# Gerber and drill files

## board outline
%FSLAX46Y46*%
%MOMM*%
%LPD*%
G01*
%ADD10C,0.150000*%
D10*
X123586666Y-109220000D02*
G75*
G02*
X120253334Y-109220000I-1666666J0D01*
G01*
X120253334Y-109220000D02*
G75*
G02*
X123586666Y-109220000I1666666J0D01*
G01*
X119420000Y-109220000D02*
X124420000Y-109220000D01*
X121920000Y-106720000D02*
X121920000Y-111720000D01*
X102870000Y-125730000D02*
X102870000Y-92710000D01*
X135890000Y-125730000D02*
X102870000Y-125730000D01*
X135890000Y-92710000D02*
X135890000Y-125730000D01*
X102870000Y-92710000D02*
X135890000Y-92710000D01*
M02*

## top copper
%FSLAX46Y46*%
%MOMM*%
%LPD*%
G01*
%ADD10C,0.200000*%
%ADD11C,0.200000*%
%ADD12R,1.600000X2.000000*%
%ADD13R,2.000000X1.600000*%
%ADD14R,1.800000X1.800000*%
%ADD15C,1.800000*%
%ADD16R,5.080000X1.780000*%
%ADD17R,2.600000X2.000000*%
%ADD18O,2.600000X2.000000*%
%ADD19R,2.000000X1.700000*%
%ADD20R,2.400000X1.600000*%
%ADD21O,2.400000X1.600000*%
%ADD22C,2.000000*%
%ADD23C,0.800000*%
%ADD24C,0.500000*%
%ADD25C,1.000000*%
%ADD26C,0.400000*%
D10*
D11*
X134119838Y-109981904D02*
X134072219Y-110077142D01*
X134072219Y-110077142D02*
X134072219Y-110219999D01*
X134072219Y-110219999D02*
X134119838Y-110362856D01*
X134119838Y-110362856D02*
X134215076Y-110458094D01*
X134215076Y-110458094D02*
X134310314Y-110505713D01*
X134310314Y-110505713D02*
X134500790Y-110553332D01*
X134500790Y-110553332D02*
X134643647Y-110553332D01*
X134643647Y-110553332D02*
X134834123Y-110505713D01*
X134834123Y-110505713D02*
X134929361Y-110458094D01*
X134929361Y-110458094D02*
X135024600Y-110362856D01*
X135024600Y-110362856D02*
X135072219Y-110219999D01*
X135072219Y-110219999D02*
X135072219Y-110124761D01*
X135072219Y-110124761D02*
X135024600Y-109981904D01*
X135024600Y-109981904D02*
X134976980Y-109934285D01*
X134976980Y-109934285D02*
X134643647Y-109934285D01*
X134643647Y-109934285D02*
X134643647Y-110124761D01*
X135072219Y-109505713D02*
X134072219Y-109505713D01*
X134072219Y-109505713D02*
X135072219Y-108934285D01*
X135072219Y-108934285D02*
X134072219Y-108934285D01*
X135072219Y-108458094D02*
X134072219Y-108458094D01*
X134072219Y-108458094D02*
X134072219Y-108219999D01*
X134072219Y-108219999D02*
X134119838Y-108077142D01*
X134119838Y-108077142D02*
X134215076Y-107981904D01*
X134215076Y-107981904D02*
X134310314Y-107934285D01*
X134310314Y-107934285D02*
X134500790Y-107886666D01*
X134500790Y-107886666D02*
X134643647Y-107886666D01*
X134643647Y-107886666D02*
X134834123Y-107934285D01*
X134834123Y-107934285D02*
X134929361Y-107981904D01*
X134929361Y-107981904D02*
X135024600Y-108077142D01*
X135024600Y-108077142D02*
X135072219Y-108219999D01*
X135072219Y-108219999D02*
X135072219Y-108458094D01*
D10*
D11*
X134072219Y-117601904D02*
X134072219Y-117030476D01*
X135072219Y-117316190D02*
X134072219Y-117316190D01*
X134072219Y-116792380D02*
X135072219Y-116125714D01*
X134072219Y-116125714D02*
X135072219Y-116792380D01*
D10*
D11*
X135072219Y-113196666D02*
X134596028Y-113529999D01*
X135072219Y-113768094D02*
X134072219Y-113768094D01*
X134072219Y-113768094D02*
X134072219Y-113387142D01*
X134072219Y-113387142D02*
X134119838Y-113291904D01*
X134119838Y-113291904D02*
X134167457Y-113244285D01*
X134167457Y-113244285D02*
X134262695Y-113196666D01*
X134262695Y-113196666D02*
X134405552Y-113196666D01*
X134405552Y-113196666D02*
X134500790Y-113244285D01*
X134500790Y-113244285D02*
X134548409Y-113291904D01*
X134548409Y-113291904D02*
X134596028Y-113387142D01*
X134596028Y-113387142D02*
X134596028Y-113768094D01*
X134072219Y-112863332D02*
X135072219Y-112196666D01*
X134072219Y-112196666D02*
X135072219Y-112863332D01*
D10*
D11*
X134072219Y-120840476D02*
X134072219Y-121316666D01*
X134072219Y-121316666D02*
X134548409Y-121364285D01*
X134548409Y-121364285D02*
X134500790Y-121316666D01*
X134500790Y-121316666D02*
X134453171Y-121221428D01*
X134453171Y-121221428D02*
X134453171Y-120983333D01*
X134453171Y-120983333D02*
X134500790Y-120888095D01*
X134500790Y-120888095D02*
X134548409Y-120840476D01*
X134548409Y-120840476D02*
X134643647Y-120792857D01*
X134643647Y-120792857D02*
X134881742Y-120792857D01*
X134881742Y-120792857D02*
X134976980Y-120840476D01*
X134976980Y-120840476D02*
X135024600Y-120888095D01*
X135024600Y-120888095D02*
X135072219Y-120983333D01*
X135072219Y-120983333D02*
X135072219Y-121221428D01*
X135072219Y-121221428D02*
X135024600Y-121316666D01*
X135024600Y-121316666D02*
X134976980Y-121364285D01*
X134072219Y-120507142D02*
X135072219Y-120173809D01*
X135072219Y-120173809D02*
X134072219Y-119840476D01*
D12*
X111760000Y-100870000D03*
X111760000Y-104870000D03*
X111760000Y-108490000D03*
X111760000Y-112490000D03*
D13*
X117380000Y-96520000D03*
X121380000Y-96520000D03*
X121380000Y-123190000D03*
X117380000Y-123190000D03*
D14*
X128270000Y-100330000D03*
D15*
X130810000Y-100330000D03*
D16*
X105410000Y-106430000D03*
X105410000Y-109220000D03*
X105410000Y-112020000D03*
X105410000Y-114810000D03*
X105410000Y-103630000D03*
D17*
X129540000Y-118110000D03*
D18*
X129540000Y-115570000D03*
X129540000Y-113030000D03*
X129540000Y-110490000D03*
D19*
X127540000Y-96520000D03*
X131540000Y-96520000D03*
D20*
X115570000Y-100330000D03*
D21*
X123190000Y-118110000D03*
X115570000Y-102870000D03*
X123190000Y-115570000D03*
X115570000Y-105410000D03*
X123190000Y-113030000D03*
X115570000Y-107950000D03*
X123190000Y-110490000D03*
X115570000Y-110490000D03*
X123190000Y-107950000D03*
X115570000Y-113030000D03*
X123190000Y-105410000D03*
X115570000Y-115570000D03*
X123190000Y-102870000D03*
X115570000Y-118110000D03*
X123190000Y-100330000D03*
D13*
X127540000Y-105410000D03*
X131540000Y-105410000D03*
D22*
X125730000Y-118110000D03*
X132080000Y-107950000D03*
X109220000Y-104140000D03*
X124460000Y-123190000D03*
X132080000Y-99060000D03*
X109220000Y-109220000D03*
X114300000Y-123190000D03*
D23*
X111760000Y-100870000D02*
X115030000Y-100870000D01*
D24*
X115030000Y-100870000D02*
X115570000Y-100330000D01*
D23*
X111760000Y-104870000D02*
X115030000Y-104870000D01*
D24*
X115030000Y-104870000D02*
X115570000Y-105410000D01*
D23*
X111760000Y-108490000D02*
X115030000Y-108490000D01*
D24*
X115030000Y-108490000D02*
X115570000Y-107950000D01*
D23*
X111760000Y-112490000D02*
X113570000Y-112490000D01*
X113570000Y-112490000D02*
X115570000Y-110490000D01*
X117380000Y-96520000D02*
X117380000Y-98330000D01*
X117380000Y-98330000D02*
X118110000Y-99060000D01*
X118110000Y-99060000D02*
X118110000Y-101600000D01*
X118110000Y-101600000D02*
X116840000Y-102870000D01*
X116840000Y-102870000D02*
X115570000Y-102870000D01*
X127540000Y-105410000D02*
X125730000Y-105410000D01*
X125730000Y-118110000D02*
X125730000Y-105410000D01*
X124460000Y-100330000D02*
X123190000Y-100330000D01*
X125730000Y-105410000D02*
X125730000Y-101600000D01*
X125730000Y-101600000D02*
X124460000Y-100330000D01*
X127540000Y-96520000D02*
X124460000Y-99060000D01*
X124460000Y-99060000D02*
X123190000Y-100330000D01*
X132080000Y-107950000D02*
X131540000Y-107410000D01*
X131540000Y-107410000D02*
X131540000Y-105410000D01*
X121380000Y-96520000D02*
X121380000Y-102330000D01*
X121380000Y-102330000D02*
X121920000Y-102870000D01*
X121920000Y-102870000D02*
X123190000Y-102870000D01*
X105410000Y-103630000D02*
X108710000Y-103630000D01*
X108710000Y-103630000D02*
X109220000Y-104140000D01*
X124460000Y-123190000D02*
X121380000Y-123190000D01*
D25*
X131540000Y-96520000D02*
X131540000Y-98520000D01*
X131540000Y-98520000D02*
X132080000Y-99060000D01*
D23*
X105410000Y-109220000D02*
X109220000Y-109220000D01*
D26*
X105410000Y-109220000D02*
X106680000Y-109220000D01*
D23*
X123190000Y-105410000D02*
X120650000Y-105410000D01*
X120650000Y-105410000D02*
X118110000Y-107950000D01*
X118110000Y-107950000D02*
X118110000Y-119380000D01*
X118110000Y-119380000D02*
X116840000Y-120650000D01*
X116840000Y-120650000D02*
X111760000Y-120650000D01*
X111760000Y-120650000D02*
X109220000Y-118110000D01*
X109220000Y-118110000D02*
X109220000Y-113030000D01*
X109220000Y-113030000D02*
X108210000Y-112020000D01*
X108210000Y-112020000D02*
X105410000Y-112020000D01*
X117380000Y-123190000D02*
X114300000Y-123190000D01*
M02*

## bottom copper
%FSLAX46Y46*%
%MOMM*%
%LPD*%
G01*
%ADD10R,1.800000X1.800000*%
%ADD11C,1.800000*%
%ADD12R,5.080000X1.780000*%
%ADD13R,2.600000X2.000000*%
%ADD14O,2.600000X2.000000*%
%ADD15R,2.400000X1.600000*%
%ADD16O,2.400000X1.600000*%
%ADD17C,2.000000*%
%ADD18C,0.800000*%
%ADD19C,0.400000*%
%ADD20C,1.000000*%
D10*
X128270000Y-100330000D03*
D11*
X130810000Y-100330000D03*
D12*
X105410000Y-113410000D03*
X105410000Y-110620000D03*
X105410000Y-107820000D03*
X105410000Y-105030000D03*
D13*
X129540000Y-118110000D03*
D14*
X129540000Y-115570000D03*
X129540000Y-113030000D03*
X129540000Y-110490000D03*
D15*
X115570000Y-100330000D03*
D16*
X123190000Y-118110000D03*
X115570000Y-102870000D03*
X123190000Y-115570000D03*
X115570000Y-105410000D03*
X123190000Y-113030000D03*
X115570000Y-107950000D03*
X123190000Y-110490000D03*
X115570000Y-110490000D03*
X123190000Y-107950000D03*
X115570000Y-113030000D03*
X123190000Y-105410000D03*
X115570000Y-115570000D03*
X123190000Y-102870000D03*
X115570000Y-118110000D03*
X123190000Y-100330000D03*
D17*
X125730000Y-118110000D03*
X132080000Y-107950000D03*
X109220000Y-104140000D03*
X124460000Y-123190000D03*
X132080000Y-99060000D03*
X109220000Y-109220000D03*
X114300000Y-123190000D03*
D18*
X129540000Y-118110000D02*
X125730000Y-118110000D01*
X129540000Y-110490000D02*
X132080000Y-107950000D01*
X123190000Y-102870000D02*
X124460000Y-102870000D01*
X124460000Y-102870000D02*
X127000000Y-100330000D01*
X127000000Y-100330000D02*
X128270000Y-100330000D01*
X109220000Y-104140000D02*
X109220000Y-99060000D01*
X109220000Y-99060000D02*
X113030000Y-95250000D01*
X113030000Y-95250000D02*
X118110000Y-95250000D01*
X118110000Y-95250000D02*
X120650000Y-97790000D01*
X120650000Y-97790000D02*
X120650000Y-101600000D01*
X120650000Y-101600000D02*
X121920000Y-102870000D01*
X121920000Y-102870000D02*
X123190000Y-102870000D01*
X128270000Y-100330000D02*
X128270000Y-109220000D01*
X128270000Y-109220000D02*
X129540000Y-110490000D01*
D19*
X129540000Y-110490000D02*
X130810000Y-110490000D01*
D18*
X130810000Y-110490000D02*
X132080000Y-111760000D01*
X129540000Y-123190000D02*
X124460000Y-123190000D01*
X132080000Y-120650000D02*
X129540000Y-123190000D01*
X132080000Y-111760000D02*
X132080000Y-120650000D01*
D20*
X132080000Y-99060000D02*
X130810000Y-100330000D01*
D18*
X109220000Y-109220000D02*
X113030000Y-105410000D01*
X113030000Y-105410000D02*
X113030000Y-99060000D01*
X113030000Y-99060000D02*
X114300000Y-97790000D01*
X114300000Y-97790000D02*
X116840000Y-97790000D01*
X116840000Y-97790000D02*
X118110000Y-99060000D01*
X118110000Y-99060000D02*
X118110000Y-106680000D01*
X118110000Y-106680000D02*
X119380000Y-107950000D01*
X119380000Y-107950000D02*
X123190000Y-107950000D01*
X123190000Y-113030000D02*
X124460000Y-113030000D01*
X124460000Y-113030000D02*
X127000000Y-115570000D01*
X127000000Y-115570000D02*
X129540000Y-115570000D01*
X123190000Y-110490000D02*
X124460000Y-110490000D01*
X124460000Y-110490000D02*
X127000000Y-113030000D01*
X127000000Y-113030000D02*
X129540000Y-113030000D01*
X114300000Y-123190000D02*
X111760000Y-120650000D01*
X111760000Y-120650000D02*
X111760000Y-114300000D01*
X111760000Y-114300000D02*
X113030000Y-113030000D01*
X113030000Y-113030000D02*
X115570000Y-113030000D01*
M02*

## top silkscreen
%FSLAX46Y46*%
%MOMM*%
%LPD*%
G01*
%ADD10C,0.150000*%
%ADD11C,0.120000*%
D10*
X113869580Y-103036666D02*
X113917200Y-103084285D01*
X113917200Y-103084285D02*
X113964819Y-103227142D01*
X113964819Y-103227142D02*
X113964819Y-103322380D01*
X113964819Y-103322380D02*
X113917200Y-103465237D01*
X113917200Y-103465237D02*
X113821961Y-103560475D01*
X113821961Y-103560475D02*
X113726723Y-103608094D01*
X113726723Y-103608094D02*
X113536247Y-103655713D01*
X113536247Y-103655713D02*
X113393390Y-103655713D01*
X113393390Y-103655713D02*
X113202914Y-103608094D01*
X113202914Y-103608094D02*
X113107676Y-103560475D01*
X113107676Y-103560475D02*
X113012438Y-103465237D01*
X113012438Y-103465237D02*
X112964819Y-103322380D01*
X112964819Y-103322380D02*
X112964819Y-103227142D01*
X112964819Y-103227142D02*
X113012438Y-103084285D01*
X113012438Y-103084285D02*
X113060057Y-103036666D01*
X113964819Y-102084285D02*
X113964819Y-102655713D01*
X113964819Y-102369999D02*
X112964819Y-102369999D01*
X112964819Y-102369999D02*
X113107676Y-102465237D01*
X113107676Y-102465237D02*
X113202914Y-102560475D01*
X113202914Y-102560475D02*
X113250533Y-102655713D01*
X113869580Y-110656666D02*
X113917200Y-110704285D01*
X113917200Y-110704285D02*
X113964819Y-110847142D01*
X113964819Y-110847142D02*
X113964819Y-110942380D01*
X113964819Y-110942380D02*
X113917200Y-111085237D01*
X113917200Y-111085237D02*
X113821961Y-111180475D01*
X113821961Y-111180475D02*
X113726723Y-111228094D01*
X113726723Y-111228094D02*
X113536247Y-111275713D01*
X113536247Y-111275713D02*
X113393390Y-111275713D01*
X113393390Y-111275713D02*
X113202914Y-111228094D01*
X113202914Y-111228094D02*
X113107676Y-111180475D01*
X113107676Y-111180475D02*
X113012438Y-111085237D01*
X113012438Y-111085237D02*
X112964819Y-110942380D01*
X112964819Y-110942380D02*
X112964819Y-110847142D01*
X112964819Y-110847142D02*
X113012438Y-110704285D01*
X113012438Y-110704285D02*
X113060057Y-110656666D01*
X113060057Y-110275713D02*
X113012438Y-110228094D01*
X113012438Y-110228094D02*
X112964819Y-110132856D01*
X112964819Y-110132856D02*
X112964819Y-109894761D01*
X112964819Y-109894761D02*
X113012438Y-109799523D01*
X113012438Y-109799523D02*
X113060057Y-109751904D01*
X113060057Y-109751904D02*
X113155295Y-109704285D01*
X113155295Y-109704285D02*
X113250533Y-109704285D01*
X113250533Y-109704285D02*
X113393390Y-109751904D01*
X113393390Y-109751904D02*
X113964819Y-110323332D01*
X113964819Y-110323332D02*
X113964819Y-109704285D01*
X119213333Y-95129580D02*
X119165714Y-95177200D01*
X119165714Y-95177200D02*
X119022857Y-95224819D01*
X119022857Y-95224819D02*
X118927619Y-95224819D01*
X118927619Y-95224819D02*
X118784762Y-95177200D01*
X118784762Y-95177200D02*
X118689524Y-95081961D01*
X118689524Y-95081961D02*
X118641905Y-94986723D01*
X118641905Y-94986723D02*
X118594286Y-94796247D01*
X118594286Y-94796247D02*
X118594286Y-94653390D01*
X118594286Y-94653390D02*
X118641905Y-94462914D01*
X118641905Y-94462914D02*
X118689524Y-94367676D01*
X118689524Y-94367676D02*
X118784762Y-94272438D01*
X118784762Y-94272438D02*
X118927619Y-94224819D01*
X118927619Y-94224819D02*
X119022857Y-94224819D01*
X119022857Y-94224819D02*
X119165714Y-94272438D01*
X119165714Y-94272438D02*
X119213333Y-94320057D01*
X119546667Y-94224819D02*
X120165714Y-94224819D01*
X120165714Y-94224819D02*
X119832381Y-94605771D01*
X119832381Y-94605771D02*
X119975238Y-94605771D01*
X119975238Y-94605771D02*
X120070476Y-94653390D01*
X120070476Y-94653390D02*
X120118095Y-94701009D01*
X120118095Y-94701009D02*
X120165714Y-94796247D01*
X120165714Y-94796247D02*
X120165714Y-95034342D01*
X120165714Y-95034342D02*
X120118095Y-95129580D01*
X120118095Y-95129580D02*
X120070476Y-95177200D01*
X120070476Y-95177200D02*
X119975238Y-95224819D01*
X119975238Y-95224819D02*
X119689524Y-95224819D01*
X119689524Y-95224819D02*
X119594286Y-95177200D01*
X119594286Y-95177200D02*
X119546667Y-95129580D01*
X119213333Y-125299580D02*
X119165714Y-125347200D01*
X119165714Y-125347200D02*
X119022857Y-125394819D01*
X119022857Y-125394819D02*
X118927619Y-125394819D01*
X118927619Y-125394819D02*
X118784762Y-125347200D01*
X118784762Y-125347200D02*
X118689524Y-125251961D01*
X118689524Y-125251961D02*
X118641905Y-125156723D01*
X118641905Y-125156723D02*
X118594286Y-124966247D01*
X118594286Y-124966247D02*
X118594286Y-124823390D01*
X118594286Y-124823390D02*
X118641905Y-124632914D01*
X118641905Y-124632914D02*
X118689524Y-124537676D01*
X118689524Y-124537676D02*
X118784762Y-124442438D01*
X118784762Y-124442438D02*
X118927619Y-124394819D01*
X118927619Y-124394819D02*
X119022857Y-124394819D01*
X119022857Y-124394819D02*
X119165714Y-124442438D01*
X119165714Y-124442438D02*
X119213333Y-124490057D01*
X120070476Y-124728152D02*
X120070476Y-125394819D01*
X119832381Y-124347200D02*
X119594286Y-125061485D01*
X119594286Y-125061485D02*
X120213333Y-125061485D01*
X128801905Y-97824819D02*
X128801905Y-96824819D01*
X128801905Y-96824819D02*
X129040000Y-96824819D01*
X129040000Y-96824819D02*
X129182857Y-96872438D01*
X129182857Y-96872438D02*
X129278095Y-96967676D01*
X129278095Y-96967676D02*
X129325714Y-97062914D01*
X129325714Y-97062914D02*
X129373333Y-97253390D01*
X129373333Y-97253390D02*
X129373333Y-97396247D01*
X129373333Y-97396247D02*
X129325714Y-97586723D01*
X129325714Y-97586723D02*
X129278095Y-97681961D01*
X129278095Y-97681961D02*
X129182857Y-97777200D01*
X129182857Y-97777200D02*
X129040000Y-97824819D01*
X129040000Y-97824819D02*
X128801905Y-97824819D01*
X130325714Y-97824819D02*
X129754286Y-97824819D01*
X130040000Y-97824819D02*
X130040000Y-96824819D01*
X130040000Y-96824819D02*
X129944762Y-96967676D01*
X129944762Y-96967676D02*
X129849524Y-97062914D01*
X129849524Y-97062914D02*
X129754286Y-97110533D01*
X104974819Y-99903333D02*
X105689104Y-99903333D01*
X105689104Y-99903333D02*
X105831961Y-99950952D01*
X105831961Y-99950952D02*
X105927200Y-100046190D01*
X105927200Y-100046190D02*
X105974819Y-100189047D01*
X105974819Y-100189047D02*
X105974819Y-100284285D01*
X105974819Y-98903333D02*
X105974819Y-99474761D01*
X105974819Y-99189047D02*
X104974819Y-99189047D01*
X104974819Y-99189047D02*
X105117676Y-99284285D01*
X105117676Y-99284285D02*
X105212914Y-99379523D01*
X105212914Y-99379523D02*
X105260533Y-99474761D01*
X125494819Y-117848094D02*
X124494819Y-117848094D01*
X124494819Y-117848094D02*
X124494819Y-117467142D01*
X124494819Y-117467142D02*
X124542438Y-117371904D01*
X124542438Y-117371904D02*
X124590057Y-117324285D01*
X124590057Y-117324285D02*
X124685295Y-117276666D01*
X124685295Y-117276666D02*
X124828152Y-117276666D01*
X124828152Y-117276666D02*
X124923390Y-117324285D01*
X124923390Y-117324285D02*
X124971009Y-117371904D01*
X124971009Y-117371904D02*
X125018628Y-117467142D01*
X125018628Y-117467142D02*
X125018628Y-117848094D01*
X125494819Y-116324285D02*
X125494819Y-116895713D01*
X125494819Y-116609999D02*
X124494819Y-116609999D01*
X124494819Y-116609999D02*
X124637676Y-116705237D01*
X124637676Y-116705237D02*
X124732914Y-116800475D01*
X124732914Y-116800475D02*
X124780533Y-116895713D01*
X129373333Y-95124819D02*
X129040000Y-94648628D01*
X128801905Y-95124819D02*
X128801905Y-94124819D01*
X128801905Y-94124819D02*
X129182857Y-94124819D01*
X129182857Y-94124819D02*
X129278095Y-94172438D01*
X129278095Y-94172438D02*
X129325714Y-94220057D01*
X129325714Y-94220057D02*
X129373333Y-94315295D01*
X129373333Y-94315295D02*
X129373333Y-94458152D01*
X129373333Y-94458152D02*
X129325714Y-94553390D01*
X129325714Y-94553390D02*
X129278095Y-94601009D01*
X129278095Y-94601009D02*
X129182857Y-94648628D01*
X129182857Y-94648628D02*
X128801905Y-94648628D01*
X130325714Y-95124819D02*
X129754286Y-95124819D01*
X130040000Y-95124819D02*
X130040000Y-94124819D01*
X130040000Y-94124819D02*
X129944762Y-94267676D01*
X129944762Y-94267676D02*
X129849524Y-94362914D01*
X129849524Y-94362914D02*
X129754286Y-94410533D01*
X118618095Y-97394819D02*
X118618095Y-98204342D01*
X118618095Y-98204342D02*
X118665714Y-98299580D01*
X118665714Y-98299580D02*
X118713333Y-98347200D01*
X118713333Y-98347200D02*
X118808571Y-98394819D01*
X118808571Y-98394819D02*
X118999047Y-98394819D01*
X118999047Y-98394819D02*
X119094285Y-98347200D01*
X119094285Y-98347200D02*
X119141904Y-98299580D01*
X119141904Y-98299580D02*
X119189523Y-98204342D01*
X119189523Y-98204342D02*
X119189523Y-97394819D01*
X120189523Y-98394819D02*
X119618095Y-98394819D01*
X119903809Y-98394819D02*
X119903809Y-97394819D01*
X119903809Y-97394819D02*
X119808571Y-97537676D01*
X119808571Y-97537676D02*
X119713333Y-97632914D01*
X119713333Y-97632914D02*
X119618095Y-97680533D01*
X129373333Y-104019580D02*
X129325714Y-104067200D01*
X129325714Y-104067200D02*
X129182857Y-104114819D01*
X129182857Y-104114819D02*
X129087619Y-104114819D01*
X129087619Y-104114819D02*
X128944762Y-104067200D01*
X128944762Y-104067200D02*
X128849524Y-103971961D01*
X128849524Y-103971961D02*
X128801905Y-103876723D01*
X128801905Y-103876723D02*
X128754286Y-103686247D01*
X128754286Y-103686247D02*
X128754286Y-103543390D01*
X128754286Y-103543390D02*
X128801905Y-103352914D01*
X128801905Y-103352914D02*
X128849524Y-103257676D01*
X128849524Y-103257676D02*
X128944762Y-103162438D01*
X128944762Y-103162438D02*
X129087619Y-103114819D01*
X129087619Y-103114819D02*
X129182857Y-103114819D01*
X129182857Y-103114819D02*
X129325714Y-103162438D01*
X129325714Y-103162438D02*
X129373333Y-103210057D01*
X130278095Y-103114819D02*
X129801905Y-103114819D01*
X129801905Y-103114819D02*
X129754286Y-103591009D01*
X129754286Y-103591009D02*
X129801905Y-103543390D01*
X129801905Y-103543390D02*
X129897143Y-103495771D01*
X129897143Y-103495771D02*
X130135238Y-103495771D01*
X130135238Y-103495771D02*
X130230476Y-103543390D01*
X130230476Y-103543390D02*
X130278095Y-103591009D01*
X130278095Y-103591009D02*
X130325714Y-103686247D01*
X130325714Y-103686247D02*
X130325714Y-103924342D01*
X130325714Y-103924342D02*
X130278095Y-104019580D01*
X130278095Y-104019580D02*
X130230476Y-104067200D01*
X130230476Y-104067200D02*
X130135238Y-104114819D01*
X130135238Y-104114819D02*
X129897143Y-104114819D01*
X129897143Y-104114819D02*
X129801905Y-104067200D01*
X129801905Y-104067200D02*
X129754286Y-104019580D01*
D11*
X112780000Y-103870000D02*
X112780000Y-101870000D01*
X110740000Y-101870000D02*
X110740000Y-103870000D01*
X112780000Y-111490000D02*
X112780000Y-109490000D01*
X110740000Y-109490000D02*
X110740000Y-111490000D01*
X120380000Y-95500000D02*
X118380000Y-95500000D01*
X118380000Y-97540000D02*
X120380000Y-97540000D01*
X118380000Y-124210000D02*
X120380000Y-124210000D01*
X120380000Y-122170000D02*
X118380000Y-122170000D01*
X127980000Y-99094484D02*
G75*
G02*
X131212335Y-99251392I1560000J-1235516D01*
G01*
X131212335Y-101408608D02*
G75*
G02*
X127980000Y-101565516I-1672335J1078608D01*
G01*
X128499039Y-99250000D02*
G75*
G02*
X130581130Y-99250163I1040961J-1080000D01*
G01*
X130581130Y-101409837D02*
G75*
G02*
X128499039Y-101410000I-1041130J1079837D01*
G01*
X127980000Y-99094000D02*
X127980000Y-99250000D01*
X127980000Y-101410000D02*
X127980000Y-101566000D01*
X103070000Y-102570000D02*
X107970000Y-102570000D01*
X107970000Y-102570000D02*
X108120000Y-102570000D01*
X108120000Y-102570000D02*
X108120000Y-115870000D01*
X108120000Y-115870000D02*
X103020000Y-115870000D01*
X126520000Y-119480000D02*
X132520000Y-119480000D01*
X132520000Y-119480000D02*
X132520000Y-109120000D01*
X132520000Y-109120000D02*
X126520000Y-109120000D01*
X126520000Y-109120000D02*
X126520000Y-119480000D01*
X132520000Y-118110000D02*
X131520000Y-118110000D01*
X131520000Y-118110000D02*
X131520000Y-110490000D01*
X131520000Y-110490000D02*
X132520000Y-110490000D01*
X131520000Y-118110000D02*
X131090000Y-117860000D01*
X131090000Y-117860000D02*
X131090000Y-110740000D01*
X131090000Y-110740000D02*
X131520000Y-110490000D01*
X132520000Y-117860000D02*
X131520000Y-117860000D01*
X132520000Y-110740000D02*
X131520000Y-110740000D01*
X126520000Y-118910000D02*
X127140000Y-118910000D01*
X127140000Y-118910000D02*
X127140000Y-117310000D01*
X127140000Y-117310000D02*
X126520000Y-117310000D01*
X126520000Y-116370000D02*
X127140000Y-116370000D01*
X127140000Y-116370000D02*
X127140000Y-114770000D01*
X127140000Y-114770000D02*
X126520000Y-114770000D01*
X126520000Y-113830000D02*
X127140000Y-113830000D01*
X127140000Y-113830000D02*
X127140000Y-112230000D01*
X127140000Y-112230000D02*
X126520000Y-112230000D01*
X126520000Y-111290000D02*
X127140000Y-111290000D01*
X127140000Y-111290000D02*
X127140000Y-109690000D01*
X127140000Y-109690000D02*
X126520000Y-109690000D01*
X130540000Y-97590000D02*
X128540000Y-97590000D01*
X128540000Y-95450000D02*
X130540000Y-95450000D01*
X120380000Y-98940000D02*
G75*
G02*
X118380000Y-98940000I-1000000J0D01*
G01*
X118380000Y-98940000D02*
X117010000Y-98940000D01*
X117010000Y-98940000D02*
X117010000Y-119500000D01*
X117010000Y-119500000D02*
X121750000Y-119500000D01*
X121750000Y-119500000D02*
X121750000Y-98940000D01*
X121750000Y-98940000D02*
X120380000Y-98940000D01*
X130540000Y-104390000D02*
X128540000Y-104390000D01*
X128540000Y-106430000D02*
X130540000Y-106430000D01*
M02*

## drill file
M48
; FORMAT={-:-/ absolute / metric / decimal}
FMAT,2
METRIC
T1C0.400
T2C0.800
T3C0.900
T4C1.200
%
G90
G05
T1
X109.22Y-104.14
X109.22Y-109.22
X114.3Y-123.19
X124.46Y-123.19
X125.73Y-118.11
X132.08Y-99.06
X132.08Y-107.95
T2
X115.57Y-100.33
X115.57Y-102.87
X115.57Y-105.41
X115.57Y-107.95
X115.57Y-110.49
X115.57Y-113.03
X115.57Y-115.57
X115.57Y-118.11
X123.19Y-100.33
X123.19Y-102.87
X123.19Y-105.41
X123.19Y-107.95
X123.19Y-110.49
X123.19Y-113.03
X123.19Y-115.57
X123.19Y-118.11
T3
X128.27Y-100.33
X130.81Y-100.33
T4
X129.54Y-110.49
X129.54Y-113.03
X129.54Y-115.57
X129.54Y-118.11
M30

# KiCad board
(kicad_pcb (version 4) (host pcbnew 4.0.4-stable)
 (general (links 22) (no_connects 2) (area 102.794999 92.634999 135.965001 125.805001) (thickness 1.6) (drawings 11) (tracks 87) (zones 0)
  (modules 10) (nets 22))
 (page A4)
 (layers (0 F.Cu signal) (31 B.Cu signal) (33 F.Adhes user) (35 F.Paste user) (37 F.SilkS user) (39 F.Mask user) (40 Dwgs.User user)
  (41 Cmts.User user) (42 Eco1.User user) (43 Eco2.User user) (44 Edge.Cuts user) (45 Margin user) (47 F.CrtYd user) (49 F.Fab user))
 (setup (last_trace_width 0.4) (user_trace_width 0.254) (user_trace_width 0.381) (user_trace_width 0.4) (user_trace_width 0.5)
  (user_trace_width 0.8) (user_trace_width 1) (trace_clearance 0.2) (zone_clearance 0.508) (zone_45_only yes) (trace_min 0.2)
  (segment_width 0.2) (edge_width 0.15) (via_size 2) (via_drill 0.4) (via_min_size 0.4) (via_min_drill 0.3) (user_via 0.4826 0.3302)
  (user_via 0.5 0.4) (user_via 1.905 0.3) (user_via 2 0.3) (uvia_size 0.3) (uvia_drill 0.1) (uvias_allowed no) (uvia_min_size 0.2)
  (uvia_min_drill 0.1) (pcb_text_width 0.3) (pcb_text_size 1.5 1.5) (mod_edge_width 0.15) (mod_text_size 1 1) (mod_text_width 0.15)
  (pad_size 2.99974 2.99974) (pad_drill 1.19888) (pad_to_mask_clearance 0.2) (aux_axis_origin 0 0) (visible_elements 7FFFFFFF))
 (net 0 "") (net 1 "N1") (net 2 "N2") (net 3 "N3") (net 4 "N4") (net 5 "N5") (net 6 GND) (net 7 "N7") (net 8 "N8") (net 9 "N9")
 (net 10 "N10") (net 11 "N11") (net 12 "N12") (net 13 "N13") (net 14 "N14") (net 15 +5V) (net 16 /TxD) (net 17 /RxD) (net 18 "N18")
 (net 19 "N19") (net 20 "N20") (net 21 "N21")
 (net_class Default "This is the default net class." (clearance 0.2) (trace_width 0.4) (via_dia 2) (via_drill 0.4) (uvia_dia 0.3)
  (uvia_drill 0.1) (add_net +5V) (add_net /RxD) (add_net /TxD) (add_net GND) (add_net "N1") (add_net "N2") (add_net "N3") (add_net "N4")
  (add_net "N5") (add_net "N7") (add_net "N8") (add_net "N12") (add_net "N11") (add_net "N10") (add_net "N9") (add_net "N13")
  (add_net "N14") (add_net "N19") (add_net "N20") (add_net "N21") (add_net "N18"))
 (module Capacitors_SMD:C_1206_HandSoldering (layer F.Cu) (at 111.76 102.87 270)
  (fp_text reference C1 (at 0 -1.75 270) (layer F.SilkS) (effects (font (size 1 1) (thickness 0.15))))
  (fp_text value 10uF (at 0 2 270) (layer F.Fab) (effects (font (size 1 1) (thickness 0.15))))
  (fp_line (start 1 -1.02) (end -1 -1.02) (layer F.SilkS) (width 0.12))
  (fp_line (start -1 1.02) (end 1 1.02) (layer F.SilkS) (width 0.12))
  (pad 1 smd rect (at -2 0 270) (size 2 1.6) (layers F.Cu F.Paste F.Mask) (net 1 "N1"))
  (pad 2 smd rect (at 2 0 270) (size 2 1.6) (layers F.Cu F.Paste F.Mask) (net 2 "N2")))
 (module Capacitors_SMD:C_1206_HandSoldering (layer F.Cu) (at 111.76 110.49 270)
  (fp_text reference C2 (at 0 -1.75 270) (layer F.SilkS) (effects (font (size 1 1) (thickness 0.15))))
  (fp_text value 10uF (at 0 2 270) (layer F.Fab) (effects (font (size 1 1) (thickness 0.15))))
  (fp_line (start 1 -1.02) (end -1 -1.02) (layer F.SilkS) (width 0.12))
  (fp_line (start -1 1.02) (end 1 1.02) (layer F.SilkS) (width 0.12))
  (pad 1 smd rect (at -2 0 270) (size 2 1.6) (layers F.Cu F.Paste F.Mask) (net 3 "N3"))
  (pad 2 smd rect (at 2 0 270) (size 2 1.6) (layers F.Cu F.Paste F.Mask) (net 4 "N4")))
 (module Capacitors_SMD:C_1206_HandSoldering (layer F.Cu) (at 119.38 96.52)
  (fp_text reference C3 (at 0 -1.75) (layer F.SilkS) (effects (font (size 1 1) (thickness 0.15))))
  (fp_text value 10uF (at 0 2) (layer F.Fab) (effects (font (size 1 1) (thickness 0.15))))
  (fp_line (start 1 -1.02) (end -1 -1.02) (layer F.SilkS) (width 0.12))
  (fp_line (start -1 1.02) (end 1 1.02) (layer F.SilkS) (width 0.12))
  (pad 1 smd rect (at -2 0) (size 2 1.6) (layers F.Cu F.Paste F.Mask) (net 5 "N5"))
  (pad 2 smd rect (at 2 0) (size 2 1.6) (layers F.Cu F.Paste F.Mask) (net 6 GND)))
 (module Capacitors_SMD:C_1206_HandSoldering (layer F.Cu) (at 119.38 123.19 180)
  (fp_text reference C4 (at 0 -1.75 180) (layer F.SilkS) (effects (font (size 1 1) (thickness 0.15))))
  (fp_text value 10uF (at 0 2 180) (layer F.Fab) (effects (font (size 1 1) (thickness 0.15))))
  (fp_line (start 1 -1.02) (end -1 -1.02) (layer F.SilkS) (width 0.12))
  (fp_line (start -1 1.02) (end 1 1.02) (layer F.SilkS) (width 0.12))
  (pad 1 smd rect (at -2 0 180) (size 2 1.6) (layers F.Cu F.Paste F.Mask) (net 6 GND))
  (pad 2 smd rect (at 2 0 180) (size 2 1.6) (layers F.Cu F.Paste F.Mask) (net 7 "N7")))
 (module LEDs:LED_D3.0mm (layer F.Cu) (at 128.27 100.33)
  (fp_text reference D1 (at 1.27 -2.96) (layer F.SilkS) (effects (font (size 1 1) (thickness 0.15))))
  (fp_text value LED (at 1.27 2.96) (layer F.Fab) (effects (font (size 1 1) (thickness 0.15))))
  (fp_arc (start 1.27 0) (end -0.29 -1.235516) (angle 108.8) (layer F.SilkS) (width 0.12))
  (fp_arc (start 1.27 0) (end -0.29 1.235516) (angle -108.8) (layer F.SilkS) (width 0.12))
  (fp_arc (start 1.27 0) (end 0.229039 -1.08) (angle 87.9) (layer F.SilkS) (width 0.12))
  (fp_arc (start 1.27 0) (end 0.229039 1.08) (angle -87.9) (layer F.SilkS) (width 0.12))
  (fp_line (start -0.29 -1.236) (end -0.29 -1.08) (layer F.SilkS) (width 0.12))
  (fp_line (start -0.29 1.08) (end -0.29 1.236) (layer F.SilkS) (width 0.12))
  (pad 1 thru_hole rect (at 0 0) (size 1.8 1.8) (drill 0.9) (layers *.Cu *.Mask) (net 6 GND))
  (pad 2 thru_hole circle (at 2.54 0) (size 1.8 1.8) (drill 0.9) (layers *.Cu *.Mask) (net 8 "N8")))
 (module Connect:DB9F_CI (layer F.Cu) (at 105.41 109.22 90)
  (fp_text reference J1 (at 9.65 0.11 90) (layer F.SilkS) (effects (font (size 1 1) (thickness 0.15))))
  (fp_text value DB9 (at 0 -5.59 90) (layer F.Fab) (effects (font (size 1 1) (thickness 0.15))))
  (fp_line (start 6.65 -2.34) (end 6.65 2.56) (layer F.SilkS) (width 0.12))
  (fp_line (start 6.65 2.56) (end 6.65 2.71) (layer F.SilkS) (width 0.12))
  (fp_line (start 6.65 2.71) (end -6.65 2.71) (layer F.SilkS) (width 0.12))
  (fp_line (start -6.65 2.71) (end -6.65 -2.39) (layer F.SilkS) (width 0.12))
  (pad 4 connect rect (at 2.79 0 90) (size 1.78 5.08) (layers F.Cu F.Mask) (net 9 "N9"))
  (pad 3 connect rect (at 0 0 90) (size 1.78 5.08) (layers F.Cu F.Mask) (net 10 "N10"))
  (pad 2 connect rect (at -2.8 0 90) (size 1.78 5.08) (layers F.Cu F.Mask) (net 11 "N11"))
  (pad 1 connect rect (at -5.59 0 90) (size 1.78 5.08) (layers F.Cu F.Mask) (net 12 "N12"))
  (pad 5 connect rect (at 5.59 0 90) (size 1.78 5.08) (layers F.Cu F.Mask) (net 6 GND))
  (pad 6 connect rect (at -4.19 0 90) (size 1.78 5.08) (layers B.Cu) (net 9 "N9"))
  (pad 7 connect rect (at -1.4 0 90) (size 1.78 5.08) (layers B.Cu) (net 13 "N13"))
  (pad 8 connect rect (at 1.4 0 90) (size 1.78 5.08) (layers B.Cu) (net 13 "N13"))
  (pad 9 connect rect (at 4.19 0 90) (size 1.78 5.08) (layers B.Cu) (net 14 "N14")))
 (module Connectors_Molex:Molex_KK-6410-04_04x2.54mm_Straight (layer F.Cu) (at 129.54 118.11 90)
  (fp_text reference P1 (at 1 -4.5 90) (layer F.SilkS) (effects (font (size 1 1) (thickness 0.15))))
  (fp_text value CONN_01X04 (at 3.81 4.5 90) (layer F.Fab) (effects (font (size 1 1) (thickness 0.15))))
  (fp_line (start -1.37 -3.02) (end -1.37 2.98) (layer F.SilkS) (width 0.12))
  (fp_line (start -1.37 2.98) (end 8.99 2.98) (layer F.SilkS) (width 0.12))
  (fp_line (start 8.99 2.98) (end 8.99 -3.02) (layer F.SilkS) (width 0.12))
  (fp_line (start 8.99 -3.02) (end -1.37 -3.02) (layer F.SilkS) (width 0.12))
  (fp_line (start 0 2.98) (end 0 1.98) (layer F.SilkS) (width 0.12))
  (fp_line (start 0 1.98) (end 7.62 1.98) (layer F.SilkS) (width 0.12))
  (fp_line (start 7.62 1.98) (end 7.62 2.98) (layer F.SilkS) (width 0.12))
  (fp_line (start 0 1.98) (end 0.25 1.55) (layer F.SilkS) (width 0.12))
  (fp_line (start 0.25 1.55) (end 7.37 1.55) (layer F.SilkS) (width 0.12))
  (fp_line (start 7.37 1.55) (end 7.62 1.98) (layer F.SilkS) (width 0.12))
  (fp_line (start 0.25 2.98) (end 0.25 1.98) (layer F.SilkS) (width 0.12))
  (fp_line (start 7.37 2.98) (end 7.37 1.98) (layer F.SilkS) (width 0.12))
  (fp_line (start -0.8 -3.02) (end -0.8 -2.4) (layer F.SilkS) (width 0.12))
  (fp_line (start -0.8 -2.4) (end 0.8 -2.4) (layer F.SilkS) (width 0.12))
  (fp_line (start 0.8 -2.4) (end 0.8 -3.02) (layer F.SilkS) (width 0.12))
  (fp_line (start 1.74 -3.02) (end 1.74 -2.4) (layer F.SilkS) (width 0.12))
  (fp_line (start 1.74 -2.4) (end 3.34 -2.4) (layer F.SilkS) (width 0.12))
  (fp_line (start 3.34 -2.4) (end 3.34 -3.02) (layer F.SilkS) (width 0.12))
  (fp_line (start 4.28 -3.02) (end 4.28 -2.4) (layer F.SilkS) (width 0.12))
  (fp_line (start 4.28 -2.4) (end 5.88 -2.4) (layer F.SilkS) (width 0.12))
  (fp_line (start 5.88 -2.4) (end 5.88 -3.02) (layer F.SilkS) (width 0.12))
  (fp_line (start 6.82 -3.02) (end 6.82 -2.4) (layer F.SilkS) (width 0.12))
  (fp_line (start 6.82 -2.4) (end 8.42 -2.4) (layer F.SilkS) (width 0.12))
  (fp_line (start 8.42 -2.4) (end 8.42 -3.02) (layer F.SilkS) (width 0.12))
  (pad 1 thru_hole rect (at 0 0 90) (size 2 2.6) (drill 1.2) (layers *.Cu *.Mask) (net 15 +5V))
  (pad 2 thru_hole oval (at 2.54 0 90) (size 2 2.6) (drill 1.2) (layers *.Cu *.Mask) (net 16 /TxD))
  (pad 3 thru_hole oval (at 5.08 0 90) (size 2 2.6) (drill 1.2) (layers *.Cu *.Mask) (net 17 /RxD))
  (pad 4 thru_hole oval (at 7.62 0 90) (size 2 2.6) (drill 1.2) (layers *.Cu *.Mask) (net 6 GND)))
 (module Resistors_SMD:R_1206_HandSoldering (layer F.Cu) (at 129.54 96.52)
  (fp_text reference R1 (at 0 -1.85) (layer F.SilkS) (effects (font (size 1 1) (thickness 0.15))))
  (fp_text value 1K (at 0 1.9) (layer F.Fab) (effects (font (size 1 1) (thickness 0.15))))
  (fp_line (start 1 1.07) (end -1 1.07) (layer F.SilkS) (width 0.12))
  (fp_line (start -1 -1.07) (end 1 -1.07) (layer F.SilkS) (width 0.12))
  (pad 1 smd rect (at -2 0) (size 2 1.7) (layers F.Cu F.Paste F.Mask) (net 15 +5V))
  (pad 2 smd rect (at 2 0) (size 2 1.7) (layers F.Cu F.Paste F.Mask) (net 8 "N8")))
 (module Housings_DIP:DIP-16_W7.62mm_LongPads (layer F.Cu) (at 115.57 100.33)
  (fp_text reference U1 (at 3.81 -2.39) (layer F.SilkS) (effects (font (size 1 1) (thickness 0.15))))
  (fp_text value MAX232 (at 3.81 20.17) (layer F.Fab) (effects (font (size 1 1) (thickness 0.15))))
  (fp_arc (start 3.81 -1.39) (end 2.81 -1.39) (angle -180) (layer F.SilkS) (width 0.12))
  (fp_line (start 2.81 -1.39) (end 1.44 -1.39) (layer F.SilkS) (width 0.12))
  (fp_line (start 1.44 -1.39) (end 1.44 19.17) (layer F.SilkS) (width 0.12))
  (fp_line (start 1.44 19.17) (end 6.18 19.17) (layer F.SilkS) (width 0.12))
  (fp_line (start 6.18 19.17) (end 6.18 -1.39) (layer F.SilkS) (width 0.12))
  (fp_line (start 6.18 -1.39) (end 4.81 -1.39) (layer F.SilkS) (width 0.12))
  (pad 1 thru_hole rect (at 0 0) (size 2.4 1.6) (drill 0.8) (layers *.Cu *.Mask) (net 1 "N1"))
  (pad 9 thru_hole oval (at 7.62 17.78) (size 2.4 1.6) (drill 0.8) (layers *.Cu *.Mask) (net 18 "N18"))
  (pad 2 thru_hole oval (at 0 2.54) (size 2.4 1.6) (drill 0.8) (layers *.Cu *.Mask) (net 5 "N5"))
  (pad 10 thru_hole oval (at 7.62 15.24) (size 2.4 1.6) (drill 0.8) (layers *.Cu *.Mask) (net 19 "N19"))
  (pad 3 thru_hole oval (at 0 5.08) (size 2.4 1.6) (drill 0.8) (layers *.Cu *.Mask) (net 2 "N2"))
  (pad 11 thru_hole oval (at 7.62 12.7) (size 2.4 1.6) (drill 0.8) (layers *.Cu *.Mask) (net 16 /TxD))
  (pad 4 thru_hole oval (at 0 7.62) (size 2.4 1.6) (drill 0.8) (layers *.Cu *.Mask) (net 3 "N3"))
  (pad 12 thru_hole oval (at 7.62 10.16) (size 2.4 1.6) (drill 0.8) (layers *.Cu *.Mask) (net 17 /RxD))
  (pad 5 thru_hole oval (at 0 10.16) (size 2.4 1.6) (drill 0.8) (layers *.Cu *.Mask) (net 4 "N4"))
  (pad 13 thru_hole oval (at 7.62 7.62) (size 2.4 1.6) (drill 0.8) (layers *.Cu *.Mask) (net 10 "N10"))
  (pad 6 thru_hole oval (at 0 12.7) (size 2.4 1.6) (drill 0.8) (layers *.Cu *.Mask) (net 7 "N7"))
  (pad 14 thru_hole oval (at 7.62 5.08) (size 2.4 1.6) (drill 0.8) (layers *.Cu *.Mask) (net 11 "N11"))
  (pad 7 thru_hole oval (at 0 15.24) (size 2.4 1.6) (drill 0.8) (layers *.Cu *.Mask) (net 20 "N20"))
  (pad 15 thru_hole oval (at 7.62 2.54) (size 2.4 1.6) (drill 0.8) (layers *.Cu *.Mask) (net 6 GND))
  (pad 8 thru_hole oval (at 0 17.78) (size 2.4 1.6) (drill 0.8) (layers *.Cu *.Mask) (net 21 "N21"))
  (pad 16 thru_hole oval (at 7.62 0) (size 2.4 1.6) (drill 0.8) (layers *.Cu *.Mask) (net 15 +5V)))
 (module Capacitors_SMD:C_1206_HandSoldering (layer F.Cu) (at 129.54 105.41)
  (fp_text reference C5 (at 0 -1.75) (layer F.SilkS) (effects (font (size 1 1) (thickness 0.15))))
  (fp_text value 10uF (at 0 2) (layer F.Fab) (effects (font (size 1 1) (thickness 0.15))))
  (fp_line (start 1 -1.02) (end -1 -1.02) (layer F.SilkS) (width 0.12))
  (fp_line (start -1 1.02) (end 1 1.02) (layer F.SilkS) (width 0.12))
  (pad 1 smd rect (at -2 0) (size 2 1.6) (layers F.Cu F.Paste F.Mask) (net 15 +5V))
  (pad 2 smd rect (at 2 0) (size 2 1.6) (layers F.Cu F.Paste F.Mask) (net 6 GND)))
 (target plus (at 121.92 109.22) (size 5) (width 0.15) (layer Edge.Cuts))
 (gr_line (start 102.87 125.73) (end 102.87 92.71) (angle 90) (layer Edge.Cuts) (width 0.15))
 (gr_line (start 135.89 125.73) (end 102.87 125.73) (angle 90) (layer Edge.Cuts) (width 0.15))
 (gr_line (start 135.89 92.71) (end 135.89 125.73) (angle 90) (layer Edge.Cuts) (width 0.15))
 (gr_line (start 102.87 92.71) (end 135.89 92.71) (angle 90) (layer Edge.Cuts) (width 0.15))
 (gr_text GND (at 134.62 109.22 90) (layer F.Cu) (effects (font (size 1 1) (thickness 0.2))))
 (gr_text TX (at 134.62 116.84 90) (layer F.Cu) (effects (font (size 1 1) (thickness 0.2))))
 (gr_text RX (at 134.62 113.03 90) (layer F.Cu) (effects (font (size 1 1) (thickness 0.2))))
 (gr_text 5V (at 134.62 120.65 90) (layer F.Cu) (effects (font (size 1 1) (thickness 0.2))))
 (segment (start 111.76 100.87) (end 115.03 100.87) (width 0.8) (layer F.Cu) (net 1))
 (segment (start 115.03 100.87) (end 115.57 100.33) (width 0.5) (layer F.Cu) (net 1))
 (segment (start 111.76 104.87) (end 115.03 104.87) (width 0.8) (layer F.Cu) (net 2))
 (segment (start 115.03 104.87) (end 115.57 105.41) (width 0.5) (layer F.Cu) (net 2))
 (segment (start 111.76 108.49) (end 115.03 108.49) (width 0.8) (layer F.Cu) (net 3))
 (segment (start 115.03 108.49) (end 115.57 107.95) (width 0.5) (layer F.Cu) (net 3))
 (segment (start 111.76 112.49) (end 113.57 112.49) (width 0.8) (layer F.Cu) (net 4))
 (segment (start 113.57 112.49) (end 115.57 110.49) (width 0.8) (layer F.Cu) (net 4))
 (segment (start 117.38 96.52) (end 117.38 98.33) (width 0.8) (layer F.Cu) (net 5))
 (segment (start 117.38 98.33) (end 118.11 99.06) (width 0.8) (layer F.Cu) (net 5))
 (segment (start 118.11 99.06) (end 118.11 101.6) (width 0.8) (layer F.Cu) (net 5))
 (segment (start 118.11 101.6) (end 116.84 102.87) (width 0.8) (layer F.Cu) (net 5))
 (segment (start 116.84 102.87) (end 115.57 102.87) (width 0.8) (layer F.Cu) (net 5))
 (segment (start 127.54 105.41) (end 125.73 105.41) (width 0.8) (layer F.Cu) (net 15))
 (segment (start 129.54 118.11) (end 125.73 118.11) (width 0.8) (layer B.Cu) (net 15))
 (via (at 125.73 118.11) (size 2) (drill 0.4) (layers F.Cu B.Cu) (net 15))
 (segment (start 125.73 118.11) (end 125.73 105.41) (width 0.8) (layer F.Cu) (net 15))
 (segment (start 124.46 100.33) (end 123.19 100.33) (width 0.8) (layer F.Cu) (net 15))
 (segment (start 125.73 105.41) (end 125.73 101.6) (width 0.8) (layer F.Cu) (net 15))
 (segment (start 125.73 101.6) (end 124.46 100.33) (width 0.8) (layer F.Cu) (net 15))
 (segment (start 127.54 96.52) (end 124.46 99.06) (width 0.8) (layer F.Cu) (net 15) (status 10))
 (segment (start 124.46 99.06) (end 123.19 100.33) (width 0.8) (layer F.Cu) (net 15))
 (segment (start 129.54 110.49) (end 132.08 107.95) (width 0.8) (layer B.Cu) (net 6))
 (via (at 132.08 107.95) (size 2) (drill 0.4) (layers F.Cu B.Cu) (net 6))
 (segment (start 132.08 107.95) (end 131.54 107.41) (width 0.8) (layer F.Cu) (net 6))
 (segment (start 131.54 107.41) (end 131.54 105.41) (width 0.8) (layer F.Cu) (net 6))
 (segment (start 123.19 102.87) (end 124.46 102.87) (width 0.8) (layer B.Cu) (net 6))
 (segment (start 124.46 102.87) (end 127 100.33) (width 0.8) (layer B.Cu) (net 6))
 (segment (start 127 100.33) (end 128.27 100.33) (width 0.8) (layer B.Cu) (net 6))
 (segment (start 121.38 96.52) (end 121.38 102.33) (width 0.8) (layer F.Cu) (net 6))
 (segment (start 121.38 102.33) (end 121.92 102.87) (width 0.8) (layer F.Cu) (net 6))
 (segment (start 121.92 102.87) (end 123.19 102.87) (width 0.8) (layer F.Cu) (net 6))
 (segment (start 105.41 103.63) (end 108.71 103.63) (width 0.8) (layer F.Cu) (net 6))
 (segment (start 108.71 103.63) (end 109.22 104.14) (width 0.8) (layer F.Cu) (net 6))
 (via (at 109.22 104.14) (size 2) (drill 0.4) (layers F.Cu B.Cu) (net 6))
 (segment (start 109.22 104.14) (end 109.22 99.06) (width 0.8) (layer B.Cu) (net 6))
 (segment (start 109.22 99.06) (end 113.03 95.25) (width 0.8) (layer B.Cu) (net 6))
 (segment (start 113.03 95.25) (end 118.11 95.25) (width 0.8) (layer B.Cu) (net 6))
 (segment (start 118.11 95.25) (end 120.65 97.79) (width 0.8) (layer B.Cu) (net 6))
 (segment (start 120.65 97.79) (end 120.65 101.6) (width 0.8) (layer B.Cu) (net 6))
 (segment (start 120.65 101.6) (end 121.92 102.87) (width 0.8) (layer B.Cu) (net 6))
 (segment (start 121.92 102.87) (end 123.19 102.87) (width 0.8) (layer B.Cu) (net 6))
 (segment (start 128.27 100.33) (end 128.27 109.22) (width 0.8) (layer B.Cu) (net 6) (status 10))
 (segment (start 128.27 109.22) (end 129.54 110.49) (width 0.8) (layer B.Cu) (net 6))
 (segment (start 129.54 110.49) (end 130.81 110.49) (width 0.4) (layer B.Cu) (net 6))
 (segment (start 130.81 110.49) (end 132.08 111.76) (width 0.8) (layer B.Cu) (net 6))
 (segment (start 124.46 123.19) (end 121.38 123.19) (width 0.8) (layer F.Cu) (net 6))
 (via (at 124.46 123.19) (size 2) (drill 0.4) (layers F.Cu B.Cu) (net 6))
 (segment (start 129.54 123.19) (end 124.46 123.19) (width 0.8) (layer B.Cu) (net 6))
 (segment (start 132.08 120.65) (end 129.54 123.19) (width 0.8) (layer B.Cu) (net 6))
 (segment (start 132.08 111.76) (end 132.08 120.65) (width 0.8) (layer B.Cu) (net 6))
 (segment (start 131.54 96.52) (end 131.54 98.52) (width 1) (layer F.Cu) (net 8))
 (segment (start 131.54 98.52) (end 132.08 99.06) (width 1) (layer F.Cu) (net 8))
 (via (at 132.08 99.06) (size 2) (drill 0.4) (layers F.Cu B.Cu) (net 8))
 (segment (start 132.08 99.06) (end 130.81 100.33) (width 1) (layer B.Cu) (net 8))
 (segment (start 105.41 109.22) (end 109.22 109.22) (width 0.8) (layer F.Cu) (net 10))
 (via (at 109.22 109.22) (size 2) (drill 0.4) (layers F.Cu B.Cu) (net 10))
 (segment (start 109.22 109.22) (end 113.03 105.41) (width 0.8) (layer B.Cu) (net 10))
 (segment (start 113.03 105.41) (end 113.03 99.06) (width 0.8) (layer B.Cu) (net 10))
 (segment (start 113.03 99.06) (end 114.3 97.79) (width 0.8) (layer B.Cu) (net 10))
 (segment (start 114.3 97.79) (end 116.84 97.79) (width 0.8) (layer B.Cu) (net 10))
 (segment (start 116.84 97.79) (end 118.11 99.06) (width 0.8) (layer B.Cu) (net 10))
 (segment (start 118.11 99.06) (end 118.11 106.68) (width 0.8) (layer B.Cu) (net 10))
 (segment (start 118.11 106.68) (end 119.38 107.95) (width 0.8) (layer B.Cu) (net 10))
 (segment (start 119.38 107.95) (end 123.19 107.95) (width 0.8) (layer B.Cu) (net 10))
 (segment (start 105.41 109.22) (end 106.68 109.22) (width 0.4) (layer F.Cu) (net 10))
 (segment (start 123.19 105.41) (end 120.65 105.41) (width 0.8) (layer F.Cu) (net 11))
 (segment (start 120.65 105.41) (end 118.11 107.95) (width 0.8) (layer F.Cu) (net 11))
 (segment (start 118.11 107.95) (end 118.11 119.38) (width 0.8) (layer F.Cu) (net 11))
 (segment (start 118.11 119.38) (end 116.84 120.65) (width 0.8) (layer F.Cu) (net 11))
 (segment (start 116.84 120.65) (end 111.76 120.65) (width 0.8) (layer F.Cu) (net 11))
 (segment (start 111.76 120.65) (end 109.22 118.11) (width 0.8) (layer F.Cu) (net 11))
 (segment (start 109.22 118.11) (end 109.22 113.03) (width 0.8) (layer F.Cu) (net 11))
 (segment (start 109.22 113.03) (end 108.21 112.02) (width 0.8) (layer F.Cu) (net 11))
 (segment (start 108.21 112.02) (end 105.41 112.02) (width 0.8) (layer F.Cu) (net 11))
 (segment (start 123.19 113.03) (end 124.46 113.03) (width 0.8) (layer B.Cu) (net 16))
 (segment (start 124.46 113.03) (end 127 115.57) (width 0.8) (layer B.Cu) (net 16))
 (segment (start 127 115.57) (end 129.54 115.57) (width 0.8) (layer B.Cu) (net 16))
 (segment (start 123.19 110.49) (end 124.46 110.49) (width 0.8) (layer B.Cu) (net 17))
 (segment (start 124.46 110.49) (end 127 113.03) (width 0.8) (layer B.Cu) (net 17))
 (segment (start 127 113.03) (end 129.54 113.03) (width 0.8) (layer B.Cu) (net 17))
 (segment (start 117.38 123.19) (end 114.3 123.19) (width 0.8) (layer F.Cu) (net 7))
 (via (at 114.3 123.19) (size 2) (drill 0.4) (layers F.Cu B.Cu) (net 7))
 (segment (start 114.3 123.19) (end 111.76 120.65) (width 0.8) (layer B.Cu) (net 7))
 (segment (start 111.76 120.65) (end 111.76 114.3) (width 0.8) (layer B.Cu) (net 7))
 (segment (start 111.76 114.3) (end 113.03 113.03) (width 0.8) (layer B.Cu) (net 7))
 (segment (start 113.03 113.03) (end 115.57 113.03) (width 0.8) (layer B.Cu) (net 7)))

